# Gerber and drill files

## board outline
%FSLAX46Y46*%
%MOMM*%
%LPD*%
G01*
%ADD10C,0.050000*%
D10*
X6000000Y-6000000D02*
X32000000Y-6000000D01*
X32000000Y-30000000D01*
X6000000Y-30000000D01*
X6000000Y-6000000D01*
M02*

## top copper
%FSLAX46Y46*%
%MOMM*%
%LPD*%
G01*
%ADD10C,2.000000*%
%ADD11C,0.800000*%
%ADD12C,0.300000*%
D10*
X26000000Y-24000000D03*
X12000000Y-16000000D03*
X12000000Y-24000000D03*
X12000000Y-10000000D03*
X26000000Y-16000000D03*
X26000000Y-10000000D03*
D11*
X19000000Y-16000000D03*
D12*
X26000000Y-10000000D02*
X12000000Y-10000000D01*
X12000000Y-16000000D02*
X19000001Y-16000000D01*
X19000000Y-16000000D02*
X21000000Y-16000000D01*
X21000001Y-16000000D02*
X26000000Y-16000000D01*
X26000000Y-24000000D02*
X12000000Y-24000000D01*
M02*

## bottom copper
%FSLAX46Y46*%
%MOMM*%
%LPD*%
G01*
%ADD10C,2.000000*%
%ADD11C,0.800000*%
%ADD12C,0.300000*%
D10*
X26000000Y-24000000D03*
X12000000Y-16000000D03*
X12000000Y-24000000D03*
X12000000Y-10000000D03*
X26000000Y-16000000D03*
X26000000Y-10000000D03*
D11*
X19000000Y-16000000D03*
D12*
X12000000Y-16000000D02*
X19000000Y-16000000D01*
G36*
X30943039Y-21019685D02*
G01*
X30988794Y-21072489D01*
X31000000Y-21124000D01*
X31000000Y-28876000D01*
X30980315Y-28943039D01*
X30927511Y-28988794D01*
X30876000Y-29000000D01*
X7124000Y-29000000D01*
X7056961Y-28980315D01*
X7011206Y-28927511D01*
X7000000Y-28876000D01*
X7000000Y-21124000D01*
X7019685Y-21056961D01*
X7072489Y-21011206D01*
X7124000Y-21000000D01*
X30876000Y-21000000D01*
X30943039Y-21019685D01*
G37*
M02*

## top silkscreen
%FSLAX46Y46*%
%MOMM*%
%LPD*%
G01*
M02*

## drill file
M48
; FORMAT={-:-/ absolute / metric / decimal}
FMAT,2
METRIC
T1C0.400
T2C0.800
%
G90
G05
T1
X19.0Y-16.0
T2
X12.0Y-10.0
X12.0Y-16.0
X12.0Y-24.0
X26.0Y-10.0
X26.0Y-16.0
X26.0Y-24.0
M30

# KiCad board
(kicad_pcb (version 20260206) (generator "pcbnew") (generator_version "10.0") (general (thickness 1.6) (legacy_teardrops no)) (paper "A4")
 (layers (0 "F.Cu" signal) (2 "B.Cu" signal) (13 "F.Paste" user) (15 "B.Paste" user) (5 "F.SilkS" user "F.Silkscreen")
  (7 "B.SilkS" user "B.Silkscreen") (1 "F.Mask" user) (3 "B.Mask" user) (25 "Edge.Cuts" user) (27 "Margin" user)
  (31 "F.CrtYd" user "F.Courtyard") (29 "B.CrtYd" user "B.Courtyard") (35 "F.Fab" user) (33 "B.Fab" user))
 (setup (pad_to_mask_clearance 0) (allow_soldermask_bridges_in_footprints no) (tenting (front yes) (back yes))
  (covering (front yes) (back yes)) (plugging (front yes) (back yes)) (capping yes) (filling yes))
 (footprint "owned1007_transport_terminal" (layer "F.Cu") (at 26 24)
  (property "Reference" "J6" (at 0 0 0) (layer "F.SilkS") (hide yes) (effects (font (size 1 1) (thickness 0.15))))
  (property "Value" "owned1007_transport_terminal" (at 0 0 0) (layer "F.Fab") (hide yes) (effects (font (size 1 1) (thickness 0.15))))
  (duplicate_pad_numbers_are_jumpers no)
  (pad "1" thru_hole circle (at 0 0) (size 2 2) (drill 0.8) (layers "*.Cu" "*.Mask") (remove_unused_layers no) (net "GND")))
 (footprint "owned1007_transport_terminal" (layer "F.Cu") (at 12 16)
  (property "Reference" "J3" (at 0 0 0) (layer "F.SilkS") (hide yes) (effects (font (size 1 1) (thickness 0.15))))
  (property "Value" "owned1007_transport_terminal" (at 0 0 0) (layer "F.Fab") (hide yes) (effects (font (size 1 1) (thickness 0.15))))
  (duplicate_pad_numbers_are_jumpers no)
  (pad "1" thru_hole circle (at 0 0) (size 2 2) (drill 0.8) (layers "*.Cu" "*.Mask") (remove_unused_layers no) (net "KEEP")))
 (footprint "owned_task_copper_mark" (layer "F.Cu") (at 10 28)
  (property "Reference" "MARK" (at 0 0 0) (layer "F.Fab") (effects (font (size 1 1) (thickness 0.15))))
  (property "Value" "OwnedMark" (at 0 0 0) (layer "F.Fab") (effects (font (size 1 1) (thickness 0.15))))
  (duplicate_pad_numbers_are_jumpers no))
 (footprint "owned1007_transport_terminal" (layer "F.Cu") (at 12 24)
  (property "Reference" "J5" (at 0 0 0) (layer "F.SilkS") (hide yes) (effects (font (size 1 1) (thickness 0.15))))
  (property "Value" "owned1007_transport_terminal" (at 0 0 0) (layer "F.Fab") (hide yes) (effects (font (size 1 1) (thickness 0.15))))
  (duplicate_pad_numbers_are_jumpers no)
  (pad "1" thru_hole circle (at 0 0) (size 2 2) (drill 0.8) (layers "*.Cu" "*.Mask") (remove_unused_layers no) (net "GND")))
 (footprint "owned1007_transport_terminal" (layer "F.Cu") (at 12 10)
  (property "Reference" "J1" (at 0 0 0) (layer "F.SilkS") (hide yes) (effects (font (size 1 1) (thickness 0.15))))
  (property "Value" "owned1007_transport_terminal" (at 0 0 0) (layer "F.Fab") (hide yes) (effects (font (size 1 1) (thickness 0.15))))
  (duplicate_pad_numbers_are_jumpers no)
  (pad "1" thru_hole circle (at 0 0) (size 2 2) (drill 0.8) (layers "*.Cu" "*.Mask") (remove_unused_layers no) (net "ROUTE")))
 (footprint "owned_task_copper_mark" (layer "F.Cu") (at 13 28)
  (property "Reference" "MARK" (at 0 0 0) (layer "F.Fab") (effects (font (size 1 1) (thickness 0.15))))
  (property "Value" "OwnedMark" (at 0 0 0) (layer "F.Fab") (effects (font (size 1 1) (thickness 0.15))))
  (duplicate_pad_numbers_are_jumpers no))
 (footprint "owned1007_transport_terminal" (layer "F.Cu") (at 26 16)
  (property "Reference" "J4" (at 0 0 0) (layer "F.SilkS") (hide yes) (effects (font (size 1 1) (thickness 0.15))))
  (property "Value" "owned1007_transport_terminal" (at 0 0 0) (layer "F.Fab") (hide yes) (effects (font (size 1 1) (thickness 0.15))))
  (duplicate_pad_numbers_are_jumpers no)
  (pad "1" thru_hole circle (at 0 0) (size 2 2) (drill 0.8) (layers "*.Cu" "*.Mask") (remove_unused_layers no) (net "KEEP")))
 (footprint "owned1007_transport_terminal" (layer "F.Cu") (at 26 10)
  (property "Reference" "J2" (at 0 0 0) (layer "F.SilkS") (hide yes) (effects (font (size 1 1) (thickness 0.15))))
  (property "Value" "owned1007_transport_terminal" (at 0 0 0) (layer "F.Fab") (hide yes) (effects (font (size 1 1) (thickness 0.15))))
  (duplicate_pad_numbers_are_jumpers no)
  (pad "1" thru_hole circle (at 0 0) (size 2 2) (drill 0.8) (layers "*.Cu" "*.Mask") (remove_unused_layers no) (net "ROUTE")))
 (gr_rect (start 6 6) (end 32 30) (stroke (width 0.05) (type default)) (fill no) (layer "Edge.Cuts"))
 (segment (start 26 10) (end 12 10) (width 0.3) (layer "F.Cu") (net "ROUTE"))
 (segment (start 12 16) (end 19.000001 16) (width 0.3) (layer "F.Cu") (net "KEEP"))
 (segment (start 19 16) (end 21 16) (width 0.3) (layer "F.Cu") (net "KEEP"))
 (segment (start 21.000001 16) (end 26 16) (width 0.3) (layer "F.Cu") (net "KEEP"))
 (via (at 19 16) (size 0.8) (drill 0.4) (layers "F.Cu" "B.Cu") (free yes) (capping no) (covering (front no) (back no))
  (plugging (front no) (back no)) (filling no) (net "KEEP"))
 (segment (start 12 16) (end 19 16) (width 0.3) (locked yes) (layer "B.Cu") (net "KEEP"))
 (segment (start 26 24) (end 12 24) (width 0.3) (layer "F.Cu") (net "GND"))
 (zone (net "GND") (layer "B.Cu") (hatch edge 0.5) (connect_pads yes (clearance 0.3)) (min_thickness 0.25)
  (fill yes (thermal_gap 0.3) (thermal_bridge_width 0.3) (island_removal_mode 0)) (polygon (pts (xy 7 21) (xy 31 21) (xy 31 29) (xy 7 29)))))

